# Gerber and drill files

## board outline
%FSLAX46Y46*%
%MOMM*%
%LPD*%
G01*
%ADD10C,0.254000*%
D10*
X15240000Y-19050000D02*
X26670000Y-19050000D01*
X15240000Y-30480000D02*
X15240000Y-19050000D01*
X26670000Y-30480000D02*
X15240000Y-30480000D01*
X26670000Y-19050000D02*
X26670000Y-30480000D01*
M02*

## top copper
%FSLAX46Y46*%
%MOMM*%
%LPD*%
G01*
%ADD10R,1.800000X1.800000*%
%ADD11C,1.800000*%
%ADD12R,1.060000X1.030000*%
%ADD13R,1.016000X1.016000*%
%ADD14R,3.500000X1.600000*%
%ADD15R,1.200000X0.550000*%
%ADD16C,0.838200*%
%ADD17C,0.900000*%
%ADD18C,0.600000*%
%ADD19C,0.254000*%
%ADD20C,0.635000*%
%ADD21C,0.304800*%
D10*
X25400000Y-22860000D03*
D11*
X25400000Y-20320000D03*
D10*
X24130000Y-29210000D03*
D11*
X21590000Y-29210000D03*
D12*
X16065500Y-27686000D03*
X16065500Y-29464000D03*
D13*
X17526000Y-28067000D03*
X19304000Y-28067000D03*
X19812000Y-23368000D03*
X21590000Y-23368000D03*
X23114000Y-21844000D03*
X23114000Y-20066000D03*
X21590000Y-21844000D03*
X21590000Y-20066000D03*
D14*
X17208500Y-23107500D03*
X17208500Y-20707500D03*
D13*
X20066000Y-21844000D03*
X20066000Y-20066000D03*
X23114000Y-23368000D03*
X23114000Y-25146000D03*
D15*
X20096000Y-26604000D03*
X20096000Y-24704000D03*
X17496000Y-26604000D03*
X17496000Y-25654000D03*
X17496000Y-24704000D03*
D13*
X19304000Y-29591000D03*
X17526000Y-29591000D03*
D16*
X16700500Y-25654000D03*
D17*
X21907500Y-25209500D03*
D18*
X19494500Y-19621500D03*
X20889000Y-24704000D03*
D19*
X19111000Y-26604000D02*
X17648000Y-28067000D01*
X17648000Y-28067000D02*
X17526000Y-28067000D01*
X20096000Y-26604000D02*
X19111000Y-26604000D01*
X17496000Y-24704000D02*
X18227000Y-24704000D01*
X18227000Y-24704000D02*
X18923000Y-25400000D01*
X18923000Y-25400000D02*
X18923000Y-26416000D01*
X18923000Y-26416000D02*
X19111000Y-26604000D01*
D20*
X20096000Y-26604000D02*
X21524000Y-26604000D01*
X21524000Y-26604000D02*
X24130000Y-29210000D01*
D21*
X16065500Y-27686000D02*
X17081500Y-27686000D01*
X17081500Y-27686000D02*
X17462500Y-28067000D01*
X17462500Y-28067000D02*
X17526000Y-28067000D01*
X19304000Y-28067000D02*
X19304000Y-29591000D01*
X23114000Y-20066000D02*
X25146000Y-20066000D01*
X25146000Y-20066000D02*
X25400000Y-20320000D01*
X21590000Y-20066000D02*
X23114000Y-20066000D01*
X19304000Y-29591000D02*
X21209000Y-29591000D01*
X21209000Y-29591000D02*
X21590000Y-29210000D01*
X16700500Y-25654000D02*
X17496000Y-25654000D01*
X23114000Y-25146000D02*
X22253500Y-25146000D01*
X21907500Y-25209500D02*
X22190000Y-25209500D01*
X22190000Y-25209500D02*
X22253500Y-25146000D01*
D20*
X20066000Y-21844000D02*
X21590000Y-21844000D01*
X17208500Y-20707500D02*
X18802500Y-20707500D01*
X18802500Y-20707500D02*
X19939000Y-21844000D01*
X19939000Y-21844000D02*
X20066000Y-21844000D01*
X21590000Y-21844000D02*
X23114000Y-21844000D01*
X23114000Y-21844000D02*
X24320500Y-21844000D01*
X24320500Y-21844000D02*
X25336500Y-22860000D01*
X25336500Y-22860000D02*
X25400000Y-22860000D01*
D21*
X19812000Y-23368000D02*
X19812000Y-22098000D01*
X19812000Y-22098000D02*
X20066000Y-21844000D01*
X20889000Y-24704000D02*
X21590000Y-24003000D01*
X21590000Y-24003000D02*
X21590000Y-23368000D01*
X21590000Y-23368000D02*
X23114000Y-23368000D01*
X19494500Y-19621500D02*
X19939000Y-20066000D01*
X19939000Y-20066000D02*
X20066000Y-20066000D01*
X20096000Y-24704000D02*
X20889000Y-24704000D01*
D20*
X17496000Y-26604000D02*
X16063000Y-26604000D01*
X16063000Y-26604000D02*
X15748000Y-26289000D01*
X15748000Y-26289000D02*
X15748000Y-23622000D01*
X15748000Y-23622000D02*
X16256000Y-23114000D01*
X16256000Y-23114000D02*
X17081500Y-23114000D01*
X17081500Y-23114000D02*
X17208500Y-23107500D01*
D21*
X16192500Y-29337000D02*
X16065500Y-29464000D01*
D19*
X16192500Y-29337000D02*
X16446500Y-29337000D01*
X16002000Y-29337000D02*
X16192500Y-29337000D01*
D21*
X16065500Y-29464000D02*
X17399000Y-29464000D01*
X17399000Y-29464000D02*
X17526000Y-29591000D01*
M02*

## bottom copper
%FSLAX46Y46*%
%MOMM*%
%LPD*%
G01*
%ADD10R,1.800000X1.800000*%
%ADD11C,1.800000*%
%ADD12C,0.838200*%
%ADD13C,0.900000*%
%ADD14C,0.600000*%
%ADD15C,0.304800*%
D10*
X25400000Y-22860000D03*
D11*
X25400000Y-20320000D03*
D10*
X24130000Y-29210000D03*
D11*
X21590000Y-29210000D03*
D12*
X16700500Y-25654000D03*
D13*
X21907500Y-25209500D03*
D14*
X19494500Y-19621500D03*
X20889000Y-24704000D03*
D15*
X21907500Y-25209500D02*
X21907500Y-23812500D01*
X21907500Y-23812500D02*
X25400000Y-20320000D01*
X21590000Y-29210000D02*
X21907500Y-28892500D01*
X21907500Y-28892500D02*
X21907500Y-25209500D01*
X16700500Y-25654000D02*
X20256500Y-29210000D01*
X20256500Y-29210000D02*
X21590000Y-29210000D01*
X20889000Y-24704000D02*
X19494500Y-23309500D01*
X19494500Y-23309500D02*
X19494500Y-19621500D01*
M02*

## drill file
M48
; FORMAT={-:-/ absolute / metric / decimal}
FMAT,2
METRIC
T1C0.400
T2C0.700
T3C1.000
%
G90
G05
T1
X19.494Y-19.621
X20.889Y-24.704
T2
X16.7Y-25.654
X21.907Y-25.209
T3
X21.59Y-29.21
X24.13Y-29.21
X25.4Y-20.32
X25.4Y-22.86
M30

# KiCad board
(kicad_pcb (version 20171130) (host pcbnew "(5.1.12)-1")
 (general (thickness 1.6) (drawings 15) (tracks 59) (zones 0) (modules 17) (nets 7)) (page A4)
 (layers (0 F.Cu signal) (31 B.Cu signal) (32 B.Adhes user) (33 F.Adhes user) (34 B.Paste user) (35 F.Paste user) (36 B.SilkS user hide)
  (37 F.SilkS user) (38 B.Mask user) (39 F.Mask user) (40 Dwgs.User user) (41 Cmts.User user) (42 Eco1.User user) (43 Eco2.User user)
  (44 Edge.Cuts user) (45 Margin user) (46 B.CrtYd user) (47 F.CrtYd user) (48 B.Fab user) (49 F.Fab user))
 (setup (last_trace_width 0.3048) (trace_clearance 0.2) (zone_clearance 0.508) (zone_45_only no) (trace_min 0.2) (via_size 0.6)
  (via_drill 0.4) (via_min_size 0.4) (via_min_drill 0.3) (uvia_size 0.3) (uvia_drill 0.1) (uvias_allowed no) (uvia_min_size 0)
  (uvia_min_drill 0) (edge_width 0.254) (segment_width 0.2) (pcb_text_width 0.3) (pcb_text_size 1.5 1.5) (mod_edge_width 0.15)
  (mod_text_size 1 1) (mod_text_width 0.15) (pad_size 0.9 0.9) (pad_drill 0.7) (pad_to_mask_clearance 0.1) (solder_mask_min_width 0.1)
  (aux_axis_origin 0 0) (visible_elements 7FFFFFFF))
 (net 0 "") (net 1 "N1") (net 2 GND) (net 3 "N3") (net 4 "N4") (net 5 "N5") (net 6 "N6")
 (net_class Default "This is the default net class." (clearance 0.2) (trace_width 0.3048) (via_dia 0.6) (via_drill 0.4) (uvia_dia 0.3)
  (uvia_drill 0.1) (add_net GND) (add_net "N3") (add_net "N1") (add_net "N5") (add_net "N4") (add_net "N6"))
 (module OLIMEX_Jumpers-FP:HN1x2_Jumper (layer F.Cu) (at 25.4 21.59 90)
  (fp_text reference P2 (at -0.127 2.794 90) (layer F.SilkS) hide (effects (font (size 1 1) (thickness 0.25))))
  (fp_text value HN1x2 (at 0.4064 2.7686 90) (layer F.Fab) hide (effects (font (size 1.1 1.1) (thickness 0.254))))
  (pad 1 thru_hole rect (at -1.27 0 180) (size 1.8 1.8) (drill 1) (layers *.Cu *.Mask F.SilkS) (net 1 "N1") (solder_mask_margin 0.0508)
   (solder_paste_margin -0.0508))
  (pad 2 thru_hole circle (at 1.27 0 180) (size 1.8 1.8) (drill 1) (layers *.Cu *.Mask F.SilkS) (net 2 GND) (solder_mask_margin 0.0508)
   (solder_paste_margin -0.0508)))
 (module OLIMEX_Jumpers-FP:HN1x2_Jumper (layer F.Cu) (at 22.86 29.21 180)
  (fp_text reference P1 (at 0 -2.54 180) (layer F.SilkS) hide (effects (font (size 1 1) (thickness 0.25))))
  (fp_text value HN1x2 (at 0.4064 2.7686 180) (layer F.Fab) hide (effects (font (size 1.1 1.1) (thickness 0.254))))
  (pad 1 thru_hole rect (at -1.27 0 270) (size 1.8 1.8) (drill 1) (layers *.Cu *.Mask F.SilkS) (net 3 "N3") (solder_mask_margin 0.0508)
   (solder_paste_margin -0.0508))
  (pad 2 thru_hole circle (at 1.27 0 270) (size 1.8 1.8) (drill 1) (layers *.Cu *.Mask F.SilkS) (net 2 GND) (solder_mask_margin 0.0508)
   (solder_paste_margin -0.0508)))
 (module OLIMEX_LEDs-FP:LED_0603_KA (layer F.Cu) (at 16.0655 28.575 270)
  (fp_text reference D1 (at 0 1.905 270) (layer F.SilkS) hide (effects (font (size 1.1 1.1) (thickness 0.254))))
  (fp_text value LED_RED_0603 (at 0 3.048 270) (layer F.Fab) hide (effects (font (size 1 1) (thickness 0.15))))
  (pad 2 smd rect (at -0.889 0 270) (size 1.03 1.06) (layers F.Cu F.Paste F.Mask) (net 3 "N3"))
  (pad 1 smd rect (at 0.889 0 270) (size 1.03 1.06) (layers F.Cu F.Paste F.Mask) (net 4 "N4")))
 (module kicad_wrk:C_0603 (layer F.Cu) (at 18.415 28.067)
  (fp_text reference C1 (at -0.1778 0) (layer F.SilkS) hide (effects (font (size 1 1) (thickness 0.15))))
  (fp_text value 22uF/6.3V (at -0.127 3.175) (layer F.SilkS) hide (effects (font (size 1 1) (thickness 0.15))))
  (pad 1 smd rect (at -0.889 0) (size 1.016 1.016) (layers F.Cu F.Paste F.Mask) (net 3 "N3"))
  (pad 2 smd rect (at 0.889 0) (size 1.016 1.016) (layers F.Cu F.Paste F.Mask) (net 2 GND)))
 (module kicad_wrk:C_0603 (layer F.Cu) (at 20.701 23.368)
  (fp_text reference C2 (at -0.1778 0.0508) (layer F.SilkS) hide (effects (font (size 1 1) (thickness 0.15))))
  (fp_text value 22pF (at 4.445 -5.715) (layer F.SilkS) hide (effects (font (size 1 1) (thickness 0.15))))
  (pad 1 smd rect (at -0.889 0) (size 1.016 1.016) (layers F.Cu F.Paste F.Mask) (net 1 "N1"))
  (pad 2 smd rect (at 0.889 0) (size 1.016 1.016) (layers F.Cu F.Paste F.Mask) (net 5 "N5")))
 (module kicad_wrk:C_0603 (layer F.Cu) (at 23.114 20.955 90)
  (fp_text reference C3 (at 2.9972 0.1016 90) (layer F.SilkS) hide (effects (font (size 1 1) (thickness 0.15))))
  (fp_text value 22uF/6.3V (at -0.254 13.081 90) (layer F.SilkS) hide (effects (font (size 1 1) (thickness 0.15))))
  (pad 1 smd rect (at -0.889 0 90) (size 1.016 1.016) (layers F.Cu F.Paste F.Mask) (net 1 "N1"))
  (pad 2 smd rect (at 0.889 0 90) (size 1.016 1.016) (layers F.Cu F.Paste F.Mask) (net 2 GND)))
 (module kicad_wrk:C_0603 (layer F.Cu) (at 21.59 20.955 90)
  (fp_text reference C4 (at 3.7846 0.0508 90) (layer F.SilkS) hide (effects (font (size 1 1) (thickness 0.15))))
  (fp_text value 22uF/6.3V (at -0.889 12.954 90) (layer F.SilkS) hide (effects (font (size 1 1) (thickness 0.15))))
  (pad 1 smd rect (at -0.889 0 90) (size 1.016 1.016) (layers F.Cu F.Paste F.Mask) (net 1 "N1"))
  (pad 2 smd rect (at 0.889 0 90) (size 1.016 1.016) (layers F.Cu F.Paste F.Mask) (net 2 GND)))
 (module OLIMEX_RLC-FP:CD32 (layer F.Cu) (at 17.2085 21.9075 90)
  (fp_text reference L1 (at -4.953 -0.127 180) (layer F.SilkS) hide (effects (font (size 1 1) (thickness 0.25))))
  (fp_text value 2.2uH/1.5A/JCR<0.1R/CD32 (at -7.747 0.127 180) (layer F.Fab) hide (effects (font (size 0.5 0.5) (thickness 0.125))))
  (pad 1 smd rect (at -1.2 0 180) (size 3.5 1.6) (layers F.Cu F.Paste F.Mask) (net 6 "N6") (solder_mask_margin 0.0508)
   (solder_paste_margin -0.0508) (clearance 0.0508))
  (pad 2 smd rect (at 1.2 0 180) (size 3.5 1.6) (layers F.Cu F.Paste F.Mask) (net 1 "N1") (solder_mask_margin 0.0508)
   (solder_paste_margin -0.0508) (clearance 0.0508)))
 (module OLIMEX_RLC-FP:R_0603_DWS (layer F.Cu) (at 20.066 20.955 90)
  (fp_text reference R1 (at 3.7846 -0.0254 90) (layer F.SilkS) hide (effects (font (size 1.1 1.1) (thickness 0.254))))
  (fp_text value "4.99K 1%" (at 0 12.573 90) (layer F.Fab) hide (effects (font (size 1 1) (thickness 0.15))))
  (pad 1 smd rect (at -0.889 0 90) (size 1.016 1.016) (layers F.Cu F.Paste F.Mask) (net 1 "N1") (solder_mask_margin 0.0508)
   (solder_paste_margin -0.0508) (clearance 0.0508))
  (pad 2 smd rect (at 0.889 0 90) (size 1.016 1.016) (layers F.Cu F.Paste F.Mask) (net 5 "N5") (solder_mask_margin 0.0508)
   (solder_paste_margin -0.0508) (clearance 0.0508)))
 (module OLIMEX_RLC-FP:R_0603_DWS (layer F.Cu) (at 23.114 24.257 270)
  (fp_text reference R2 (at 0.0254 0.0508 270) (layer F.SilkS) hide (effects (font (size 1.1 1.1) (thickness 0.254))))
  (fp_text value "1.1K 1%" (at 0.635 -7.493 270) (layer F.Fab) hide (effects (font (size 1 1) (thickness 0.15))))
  (pad 1 smd rect (at -0.889 0 270) (size 1.016 1.016) (layers F.Cu F.Paste F.Mask) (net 5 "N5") (solder_mask_margin 0.0508)
   (solder_paste_margin -0.0508) (clearance 0.0508))
  (pad 2 smd rect (at 0.889 0 270) (size 1.016 1.016) (layers F.Cu F.Paste F.Mask) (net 2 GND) (solder_mask_margin 0.0508)
   (solder_paste_margin -0.0508) (clearance 0.0508)))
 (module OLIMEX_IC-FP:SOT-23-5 (layer F.Cu) (at 18.796 25.654 180)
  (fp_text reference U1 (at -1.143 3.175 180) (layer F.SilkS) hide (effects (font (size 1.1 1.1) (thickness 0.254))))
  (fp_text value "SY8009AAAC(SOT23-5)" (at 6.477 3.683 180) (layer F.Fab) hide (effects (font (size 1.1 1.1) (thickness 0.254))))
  (pad 4 smd rect (at -1.3 -0.95 180) (size 1.2 0.55) (layers F.Cu F.Paste F.Mask) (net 3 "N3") (solder_mask_margin 0.0508)
   (solder_paste_margin -0.0508) (clearance 0.0508))
  (pad 5 smd rect (at -1.3 0.95 180) (size 1.2 0.55) (layers F.Cu F.Paste F.Mask) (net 5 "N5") (solder_mask_margin 0.0508)
   (solder_paste_margin -0.0508) (clearance 0.0508))
  (pad 3 smd rect (at 1.3 -0.95 180) (size 1.2 0.55) (layers F.Cu F.Paste F.Mask) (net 6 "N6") (solder_mask_margin 0.0508)
   (solder_paste_margin -0.0508) (clearance 0.0508))
  (pad 2 smd rect (at 1.3 0 180) (size 1.2 0.55) (layers F.Cu F.Paste F.Mask) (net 2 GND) (solder_mask_margin 0.0508)
   (solder_paste_margin -0.0508) (clearance 0.0508))
  (pad 1 smd rect (at 1.3 0.95 180) (size 1.2 0.55) (layers F.Cu F.Paste F.Mask) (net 3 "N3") (solder_mask_margin 0.0508)
   (solder_paste_margin -0.0508) (clearance 0.0508)))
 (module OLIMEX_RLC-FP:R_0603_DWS (layer F.Cu) (at 18.415 29.591 180)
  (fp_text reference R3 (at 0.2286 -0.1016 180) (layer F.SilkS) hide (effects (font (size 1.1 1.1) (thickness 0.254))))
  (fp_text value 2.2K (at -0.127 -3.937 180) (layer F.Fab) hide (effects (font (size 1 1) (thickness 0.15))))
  (pad 1 smd rect (at -0.889 0 180) (size 1.016 1.016) (layers F.Cu F.Paste F.Mask) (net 2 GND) (solder_mask_margin 0.0508)
   (solder_paste_margin -0.0508) (clearance 0.0508))
  (pad 2 smd rect (at 0.889 0 180) (size 1.016 1.016) (layers F.Cu F.Paste F.Mask) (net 4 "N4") (solder_mask_margin 0.0508)
   (solder_paste_margin -0.0508) (clearance 0.0508)))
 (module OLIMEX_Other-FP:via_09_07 (layer F.Cu) (at 16.7005 25.654)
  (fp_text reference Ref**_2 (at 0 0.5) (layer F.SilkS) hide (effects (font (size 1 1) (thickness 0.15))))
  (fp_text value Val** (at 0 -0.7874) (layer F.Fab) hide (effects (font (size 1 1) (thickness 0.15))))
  (pad 0 thru_hole circle (at 0 0) (size 0.8382 0.8382) (drill 0.7) (layers *.Cu) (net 2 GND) (zone_connect 2)))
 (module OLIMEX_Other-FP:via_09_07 (layer F.Cu) (at 21.9075 25.273)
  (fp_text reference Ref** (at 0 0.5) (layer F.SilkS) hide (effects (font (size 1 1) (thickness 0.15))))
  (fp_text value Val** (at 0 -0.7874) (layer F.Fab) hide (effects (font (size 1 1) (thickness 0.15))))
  (pad 0 thru_hole circle (at 0 -0.0635) (size 0.9 0.9) (drill 0.7) (layers *.Cu) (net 2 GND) (zone_connect 2)))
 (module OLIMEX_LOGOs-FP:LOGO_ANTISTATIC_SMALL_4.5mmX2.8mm (layer B.Cu) (at 18.4785 28.194 180)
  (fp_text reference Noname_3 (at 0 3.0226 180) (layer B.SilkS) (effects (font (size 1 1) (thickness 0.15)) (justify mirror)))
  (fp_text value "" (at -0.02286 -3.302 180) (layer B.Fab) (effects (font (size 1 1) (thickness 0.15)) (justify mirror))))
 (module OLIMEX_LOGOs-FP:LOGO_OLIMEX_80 (layer B.Cu) (at 19.939 24.3205 180)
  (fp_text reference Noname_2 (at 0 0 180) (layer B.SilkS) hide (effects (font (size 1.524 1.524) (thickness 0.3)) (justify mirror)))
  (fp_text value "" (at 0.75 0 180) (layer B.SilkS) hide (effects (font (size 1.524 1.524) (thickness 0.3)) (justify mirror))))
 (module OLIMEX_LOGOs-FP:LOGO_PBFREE (layer B.Cu) (at 18.669 21.3995 180)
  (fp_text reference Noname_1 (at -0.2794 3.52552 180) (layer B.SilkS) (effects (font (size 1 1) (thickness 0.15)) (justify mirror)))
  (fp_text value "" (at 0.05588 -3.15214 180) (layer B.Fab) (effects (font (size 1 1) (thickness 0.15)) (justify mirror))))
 (gr_line (start 15.24 19.05) (end 26.67 19.05) (angle 90) (layer Edge.Cuts) (width 0.254))
 (gr_line (start 15.24 30.48) (end 15.24 19.05) (angle 90) (layer Edge.Cuts) (width 0.254))
 (gr_line (start 26.67 30.48) (end 15.24 30.48) (angle 90) (layer Edge.Cuts) (width 0.254))
 (gr_line (start 26.67 19.05) (end 26.67 30.48) (angle 90) (layer Edge.Cuts) (width 0.254))
 (segment (start 19.111 26.604) (end 17.648 28.067) (width 0.254) (layer F.Cu) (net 3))
 (segment (start 17.648 28.067) (end 17.526 28.067) (width 0.254) (layer F.Cu) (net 3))
 (segment (start 20.096 26.604) (end 19.111 26.604) (width 0.254) (layer F.Cu) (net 3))
 (segment (start 17.496 24.704) (end 18.227 24.704) (width 0.254) (layer F.Cu) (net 3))
 (segment (start 18.227 24.704) (end 18.923 25.4) (width 0.254) (layer F.Cu) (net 3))
 (segment (start 18.923 25.4) (end 18.923 26.416) (width 0.254) (layer F.Cu) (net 3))
 (segment (start 18.923 26.416) (end 19.111 26.604) (width 0.254) (layer F.Cu) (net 3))
 (segment (start 20.096 26.604) (end 21.524 26.604) (width 0.635) (layer F.Cu) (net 3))
 (segment (start 21.524 26.604) (end 24.13 29.21) (width 0.635) (layer F.Cu) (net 3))
 (segment (start 16.0655 27.686) (end 17.0815 27.686) (width 0.3048) (layer F.Cu) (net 3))
 (segment (start 17.0815 27.686) (end 17.4625 28.067) (width 0.3048) (layer F.Cu) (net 3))
 (segment (start 17.4625 28.067) (end 17.526 28.067) (width 0.3048) (layer F.Cu) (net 3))
 (segment (start 21.9075 25.2095) (end 21.9075 23.8125) (width 0.3048) (layer B.Cu) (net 2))
 (segment (start 21.9075 23.8125) (end 25.4 20.32) (width 0.3048) (layer B.Cu) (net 2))
 (segment (start 21.59 29.21) (end 21.9075 28.8925) (width 0.3048) (layer B.Cu) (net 2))
 (segment (start 21.9075 28.8925) (end 21.9075 25.2095) (width 0.3048) (layer B.Cu) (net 2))
 (segment (start 19.304 28.067) (end 19.304 29.591) (width 0.3048) (layer F.Cu) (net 2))
 (segment (start 23.114 20.066) (end 25.146 20.066) (width 0.3048) (layer F.Cu) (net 2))
 (segment (start 25.146 20.066) (end 25.4 20.32) (width 0.3048) (layer F.Cu) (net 2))
 (segment (start 21.59 20.066) (end 23.114 20.066) (width 0.3048) (layer F.Cu) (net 2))
 (segment (start 19.304 29.591) (end 21.209 29.591) (width 0.3048) (layer F.Cu) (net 2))
 (segment (start 21.209 29.591) (end 21.59 29.21) (width 0.3048) (layer F.Cu) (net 2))
 (segment (start 16.7005 25.654) (end 20.2565 29.21) (width 0.3048) (layer B.Cu) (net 2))
 (segment (start 20.2565 29.21) (end 21.59 29.21) (width 0.3048) (layer B.Cu) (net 2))
 (segment (start 16.7005 25.654) (end 17.496 25.654) (width 0.3048) (layer F.Cu) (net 2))
 (segment (start 23.114 25.146) (end 22.2535 25.146) (width 0.3048) (layer F.Cu) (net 2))
 (segment (start 21.9075 25.2095) (end 22.19 25.2095) (width 0.3048) (layer F.Cu) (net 2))
 (segment (start 22.19 25.2095) (end 22.2535 25.146) (width 0.3048) (layer F.Cu) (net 2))
 (segment (start 20.066 21.844) (end 21.59 21.844) (width 0.635) (layer F.Cu) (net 1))
 (segment (start 17.2085 20.7075) (end 18.8025 20.7075) (width 0.635) (layer F.Cu) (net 1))
 (segment (start 18.8025 20.7075) (end 19.939 21.844) (width 0.635) (layer F.Cu) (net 1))
 (segment (start 19.939 21.844) (end 20.066 21.844) (width 0.635) (layer F.Cu) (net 1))
 (segment (start 21.59 21.844) (end 23.114 21.844) (width 0.635) (layer F.Cu) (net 1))
 (segment (start 23.114 21.844) (end 24.3205 21.844) (width 0.635) (layer F.Cu) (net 1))
 (segment (start 24.3205 21.844) (end 25.3365 22.86) (width 0.635) (layer F.Cu) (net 1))
 (segment (start 25.3365 22.86) (end 25.4 22.86) (width 0.635) (layer F.Cu) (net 1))
 (segment (start 19.812 23.368) (end 19.812 22.098) (width 0.3048) (layer F.Cu) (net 1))
 (segment (start 19.812 22.098) (end 20.066 21.844) (width 0.3048) (layer F.Cu) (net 1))
 (segment (start 20.889 24.704) (end 21.59 24.003) (width 0.3048) (layer F.Cu) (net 5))
 (segment (start 21.59 24.003) (end 21.59 23.368) (width 0.3048) (layer F.Cu) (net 5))
 (segment (start 21.59 23.368) (end 23.114 23.368) (width 0.3048) (layer F.Cu) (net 5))
 (segment (start 19.4945 19.6215) (end 19.939 20.066) (width 0.3048) (layer F.Cu) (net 5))
 (segment (start 19.939 20.066) (end 20.066 20.066) (width 0.3048) (layer F.Cu) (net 5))
 (segment (start 20.889 24.704) (end 19.4945 23.3095) (width 0.3048) (layer B.Cu) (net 5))
 (segment (start 19.4945 23.3095) (end 19.4945 19.6215) (width 0.3048) (layer B.Cu) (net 5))
 (segment (start 20.096 24.704) (end 20.889 24.704) (width 0.3048) (layer F.Cu) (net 5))
 (via (at 19.4945 19.6215) (size 0.6) (layers F.Cu B.Cu) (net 5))
 (via (at 20.889 24.704) (size 0.6) (layers F.Cu B.Cu) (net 5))
 (segment (start 17.496 26.604) (end 16.063 26.604) (width 0.635) (layer F.Cu) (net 6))
 (segment (start 16.063 26.604) (end 15.748 26.289) (width 0.635) (layer F.Cu) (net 6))
 (segment (start 15.748 26.289) (end 15.748 23.622) (width 0.635) (layer F.Cu) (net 6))
 (segment (start 15.748 23.622) (end 16.256 23.114) (width 0.635) (layer F.Cu) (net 6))
 (segment (start 16.256 23.114) (end 17.0815 23.114) (width 0.635) (layer F.Cu) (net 6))
 (segment (start 17.0815 23.114) (end 17.2085 23.1075) (width 0.635) (layer F.Cu) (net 6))
 (segment (start 16.1925 29.337) (end 16.0655 29.464) (width 0.3048) (layer F.Cu) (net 4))
 (segment (start 16.1925 29.337) (end 16.4465 29.337) (width 0.254) (layer F.Cu) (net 4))
 (segment (start 16.002 29.337) (end 16.1925 29.337) (width 0.254) (layer F.Cu) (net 4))
 (segment (start 16.0655 29.464) (end 17.399 29.464) (width 0.3048) (layer F.Cu) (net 4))
 (segment (start 17.399 29.464) (end 17.526 29.591) (width 0.3048) (layer F.Cu) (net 4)))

